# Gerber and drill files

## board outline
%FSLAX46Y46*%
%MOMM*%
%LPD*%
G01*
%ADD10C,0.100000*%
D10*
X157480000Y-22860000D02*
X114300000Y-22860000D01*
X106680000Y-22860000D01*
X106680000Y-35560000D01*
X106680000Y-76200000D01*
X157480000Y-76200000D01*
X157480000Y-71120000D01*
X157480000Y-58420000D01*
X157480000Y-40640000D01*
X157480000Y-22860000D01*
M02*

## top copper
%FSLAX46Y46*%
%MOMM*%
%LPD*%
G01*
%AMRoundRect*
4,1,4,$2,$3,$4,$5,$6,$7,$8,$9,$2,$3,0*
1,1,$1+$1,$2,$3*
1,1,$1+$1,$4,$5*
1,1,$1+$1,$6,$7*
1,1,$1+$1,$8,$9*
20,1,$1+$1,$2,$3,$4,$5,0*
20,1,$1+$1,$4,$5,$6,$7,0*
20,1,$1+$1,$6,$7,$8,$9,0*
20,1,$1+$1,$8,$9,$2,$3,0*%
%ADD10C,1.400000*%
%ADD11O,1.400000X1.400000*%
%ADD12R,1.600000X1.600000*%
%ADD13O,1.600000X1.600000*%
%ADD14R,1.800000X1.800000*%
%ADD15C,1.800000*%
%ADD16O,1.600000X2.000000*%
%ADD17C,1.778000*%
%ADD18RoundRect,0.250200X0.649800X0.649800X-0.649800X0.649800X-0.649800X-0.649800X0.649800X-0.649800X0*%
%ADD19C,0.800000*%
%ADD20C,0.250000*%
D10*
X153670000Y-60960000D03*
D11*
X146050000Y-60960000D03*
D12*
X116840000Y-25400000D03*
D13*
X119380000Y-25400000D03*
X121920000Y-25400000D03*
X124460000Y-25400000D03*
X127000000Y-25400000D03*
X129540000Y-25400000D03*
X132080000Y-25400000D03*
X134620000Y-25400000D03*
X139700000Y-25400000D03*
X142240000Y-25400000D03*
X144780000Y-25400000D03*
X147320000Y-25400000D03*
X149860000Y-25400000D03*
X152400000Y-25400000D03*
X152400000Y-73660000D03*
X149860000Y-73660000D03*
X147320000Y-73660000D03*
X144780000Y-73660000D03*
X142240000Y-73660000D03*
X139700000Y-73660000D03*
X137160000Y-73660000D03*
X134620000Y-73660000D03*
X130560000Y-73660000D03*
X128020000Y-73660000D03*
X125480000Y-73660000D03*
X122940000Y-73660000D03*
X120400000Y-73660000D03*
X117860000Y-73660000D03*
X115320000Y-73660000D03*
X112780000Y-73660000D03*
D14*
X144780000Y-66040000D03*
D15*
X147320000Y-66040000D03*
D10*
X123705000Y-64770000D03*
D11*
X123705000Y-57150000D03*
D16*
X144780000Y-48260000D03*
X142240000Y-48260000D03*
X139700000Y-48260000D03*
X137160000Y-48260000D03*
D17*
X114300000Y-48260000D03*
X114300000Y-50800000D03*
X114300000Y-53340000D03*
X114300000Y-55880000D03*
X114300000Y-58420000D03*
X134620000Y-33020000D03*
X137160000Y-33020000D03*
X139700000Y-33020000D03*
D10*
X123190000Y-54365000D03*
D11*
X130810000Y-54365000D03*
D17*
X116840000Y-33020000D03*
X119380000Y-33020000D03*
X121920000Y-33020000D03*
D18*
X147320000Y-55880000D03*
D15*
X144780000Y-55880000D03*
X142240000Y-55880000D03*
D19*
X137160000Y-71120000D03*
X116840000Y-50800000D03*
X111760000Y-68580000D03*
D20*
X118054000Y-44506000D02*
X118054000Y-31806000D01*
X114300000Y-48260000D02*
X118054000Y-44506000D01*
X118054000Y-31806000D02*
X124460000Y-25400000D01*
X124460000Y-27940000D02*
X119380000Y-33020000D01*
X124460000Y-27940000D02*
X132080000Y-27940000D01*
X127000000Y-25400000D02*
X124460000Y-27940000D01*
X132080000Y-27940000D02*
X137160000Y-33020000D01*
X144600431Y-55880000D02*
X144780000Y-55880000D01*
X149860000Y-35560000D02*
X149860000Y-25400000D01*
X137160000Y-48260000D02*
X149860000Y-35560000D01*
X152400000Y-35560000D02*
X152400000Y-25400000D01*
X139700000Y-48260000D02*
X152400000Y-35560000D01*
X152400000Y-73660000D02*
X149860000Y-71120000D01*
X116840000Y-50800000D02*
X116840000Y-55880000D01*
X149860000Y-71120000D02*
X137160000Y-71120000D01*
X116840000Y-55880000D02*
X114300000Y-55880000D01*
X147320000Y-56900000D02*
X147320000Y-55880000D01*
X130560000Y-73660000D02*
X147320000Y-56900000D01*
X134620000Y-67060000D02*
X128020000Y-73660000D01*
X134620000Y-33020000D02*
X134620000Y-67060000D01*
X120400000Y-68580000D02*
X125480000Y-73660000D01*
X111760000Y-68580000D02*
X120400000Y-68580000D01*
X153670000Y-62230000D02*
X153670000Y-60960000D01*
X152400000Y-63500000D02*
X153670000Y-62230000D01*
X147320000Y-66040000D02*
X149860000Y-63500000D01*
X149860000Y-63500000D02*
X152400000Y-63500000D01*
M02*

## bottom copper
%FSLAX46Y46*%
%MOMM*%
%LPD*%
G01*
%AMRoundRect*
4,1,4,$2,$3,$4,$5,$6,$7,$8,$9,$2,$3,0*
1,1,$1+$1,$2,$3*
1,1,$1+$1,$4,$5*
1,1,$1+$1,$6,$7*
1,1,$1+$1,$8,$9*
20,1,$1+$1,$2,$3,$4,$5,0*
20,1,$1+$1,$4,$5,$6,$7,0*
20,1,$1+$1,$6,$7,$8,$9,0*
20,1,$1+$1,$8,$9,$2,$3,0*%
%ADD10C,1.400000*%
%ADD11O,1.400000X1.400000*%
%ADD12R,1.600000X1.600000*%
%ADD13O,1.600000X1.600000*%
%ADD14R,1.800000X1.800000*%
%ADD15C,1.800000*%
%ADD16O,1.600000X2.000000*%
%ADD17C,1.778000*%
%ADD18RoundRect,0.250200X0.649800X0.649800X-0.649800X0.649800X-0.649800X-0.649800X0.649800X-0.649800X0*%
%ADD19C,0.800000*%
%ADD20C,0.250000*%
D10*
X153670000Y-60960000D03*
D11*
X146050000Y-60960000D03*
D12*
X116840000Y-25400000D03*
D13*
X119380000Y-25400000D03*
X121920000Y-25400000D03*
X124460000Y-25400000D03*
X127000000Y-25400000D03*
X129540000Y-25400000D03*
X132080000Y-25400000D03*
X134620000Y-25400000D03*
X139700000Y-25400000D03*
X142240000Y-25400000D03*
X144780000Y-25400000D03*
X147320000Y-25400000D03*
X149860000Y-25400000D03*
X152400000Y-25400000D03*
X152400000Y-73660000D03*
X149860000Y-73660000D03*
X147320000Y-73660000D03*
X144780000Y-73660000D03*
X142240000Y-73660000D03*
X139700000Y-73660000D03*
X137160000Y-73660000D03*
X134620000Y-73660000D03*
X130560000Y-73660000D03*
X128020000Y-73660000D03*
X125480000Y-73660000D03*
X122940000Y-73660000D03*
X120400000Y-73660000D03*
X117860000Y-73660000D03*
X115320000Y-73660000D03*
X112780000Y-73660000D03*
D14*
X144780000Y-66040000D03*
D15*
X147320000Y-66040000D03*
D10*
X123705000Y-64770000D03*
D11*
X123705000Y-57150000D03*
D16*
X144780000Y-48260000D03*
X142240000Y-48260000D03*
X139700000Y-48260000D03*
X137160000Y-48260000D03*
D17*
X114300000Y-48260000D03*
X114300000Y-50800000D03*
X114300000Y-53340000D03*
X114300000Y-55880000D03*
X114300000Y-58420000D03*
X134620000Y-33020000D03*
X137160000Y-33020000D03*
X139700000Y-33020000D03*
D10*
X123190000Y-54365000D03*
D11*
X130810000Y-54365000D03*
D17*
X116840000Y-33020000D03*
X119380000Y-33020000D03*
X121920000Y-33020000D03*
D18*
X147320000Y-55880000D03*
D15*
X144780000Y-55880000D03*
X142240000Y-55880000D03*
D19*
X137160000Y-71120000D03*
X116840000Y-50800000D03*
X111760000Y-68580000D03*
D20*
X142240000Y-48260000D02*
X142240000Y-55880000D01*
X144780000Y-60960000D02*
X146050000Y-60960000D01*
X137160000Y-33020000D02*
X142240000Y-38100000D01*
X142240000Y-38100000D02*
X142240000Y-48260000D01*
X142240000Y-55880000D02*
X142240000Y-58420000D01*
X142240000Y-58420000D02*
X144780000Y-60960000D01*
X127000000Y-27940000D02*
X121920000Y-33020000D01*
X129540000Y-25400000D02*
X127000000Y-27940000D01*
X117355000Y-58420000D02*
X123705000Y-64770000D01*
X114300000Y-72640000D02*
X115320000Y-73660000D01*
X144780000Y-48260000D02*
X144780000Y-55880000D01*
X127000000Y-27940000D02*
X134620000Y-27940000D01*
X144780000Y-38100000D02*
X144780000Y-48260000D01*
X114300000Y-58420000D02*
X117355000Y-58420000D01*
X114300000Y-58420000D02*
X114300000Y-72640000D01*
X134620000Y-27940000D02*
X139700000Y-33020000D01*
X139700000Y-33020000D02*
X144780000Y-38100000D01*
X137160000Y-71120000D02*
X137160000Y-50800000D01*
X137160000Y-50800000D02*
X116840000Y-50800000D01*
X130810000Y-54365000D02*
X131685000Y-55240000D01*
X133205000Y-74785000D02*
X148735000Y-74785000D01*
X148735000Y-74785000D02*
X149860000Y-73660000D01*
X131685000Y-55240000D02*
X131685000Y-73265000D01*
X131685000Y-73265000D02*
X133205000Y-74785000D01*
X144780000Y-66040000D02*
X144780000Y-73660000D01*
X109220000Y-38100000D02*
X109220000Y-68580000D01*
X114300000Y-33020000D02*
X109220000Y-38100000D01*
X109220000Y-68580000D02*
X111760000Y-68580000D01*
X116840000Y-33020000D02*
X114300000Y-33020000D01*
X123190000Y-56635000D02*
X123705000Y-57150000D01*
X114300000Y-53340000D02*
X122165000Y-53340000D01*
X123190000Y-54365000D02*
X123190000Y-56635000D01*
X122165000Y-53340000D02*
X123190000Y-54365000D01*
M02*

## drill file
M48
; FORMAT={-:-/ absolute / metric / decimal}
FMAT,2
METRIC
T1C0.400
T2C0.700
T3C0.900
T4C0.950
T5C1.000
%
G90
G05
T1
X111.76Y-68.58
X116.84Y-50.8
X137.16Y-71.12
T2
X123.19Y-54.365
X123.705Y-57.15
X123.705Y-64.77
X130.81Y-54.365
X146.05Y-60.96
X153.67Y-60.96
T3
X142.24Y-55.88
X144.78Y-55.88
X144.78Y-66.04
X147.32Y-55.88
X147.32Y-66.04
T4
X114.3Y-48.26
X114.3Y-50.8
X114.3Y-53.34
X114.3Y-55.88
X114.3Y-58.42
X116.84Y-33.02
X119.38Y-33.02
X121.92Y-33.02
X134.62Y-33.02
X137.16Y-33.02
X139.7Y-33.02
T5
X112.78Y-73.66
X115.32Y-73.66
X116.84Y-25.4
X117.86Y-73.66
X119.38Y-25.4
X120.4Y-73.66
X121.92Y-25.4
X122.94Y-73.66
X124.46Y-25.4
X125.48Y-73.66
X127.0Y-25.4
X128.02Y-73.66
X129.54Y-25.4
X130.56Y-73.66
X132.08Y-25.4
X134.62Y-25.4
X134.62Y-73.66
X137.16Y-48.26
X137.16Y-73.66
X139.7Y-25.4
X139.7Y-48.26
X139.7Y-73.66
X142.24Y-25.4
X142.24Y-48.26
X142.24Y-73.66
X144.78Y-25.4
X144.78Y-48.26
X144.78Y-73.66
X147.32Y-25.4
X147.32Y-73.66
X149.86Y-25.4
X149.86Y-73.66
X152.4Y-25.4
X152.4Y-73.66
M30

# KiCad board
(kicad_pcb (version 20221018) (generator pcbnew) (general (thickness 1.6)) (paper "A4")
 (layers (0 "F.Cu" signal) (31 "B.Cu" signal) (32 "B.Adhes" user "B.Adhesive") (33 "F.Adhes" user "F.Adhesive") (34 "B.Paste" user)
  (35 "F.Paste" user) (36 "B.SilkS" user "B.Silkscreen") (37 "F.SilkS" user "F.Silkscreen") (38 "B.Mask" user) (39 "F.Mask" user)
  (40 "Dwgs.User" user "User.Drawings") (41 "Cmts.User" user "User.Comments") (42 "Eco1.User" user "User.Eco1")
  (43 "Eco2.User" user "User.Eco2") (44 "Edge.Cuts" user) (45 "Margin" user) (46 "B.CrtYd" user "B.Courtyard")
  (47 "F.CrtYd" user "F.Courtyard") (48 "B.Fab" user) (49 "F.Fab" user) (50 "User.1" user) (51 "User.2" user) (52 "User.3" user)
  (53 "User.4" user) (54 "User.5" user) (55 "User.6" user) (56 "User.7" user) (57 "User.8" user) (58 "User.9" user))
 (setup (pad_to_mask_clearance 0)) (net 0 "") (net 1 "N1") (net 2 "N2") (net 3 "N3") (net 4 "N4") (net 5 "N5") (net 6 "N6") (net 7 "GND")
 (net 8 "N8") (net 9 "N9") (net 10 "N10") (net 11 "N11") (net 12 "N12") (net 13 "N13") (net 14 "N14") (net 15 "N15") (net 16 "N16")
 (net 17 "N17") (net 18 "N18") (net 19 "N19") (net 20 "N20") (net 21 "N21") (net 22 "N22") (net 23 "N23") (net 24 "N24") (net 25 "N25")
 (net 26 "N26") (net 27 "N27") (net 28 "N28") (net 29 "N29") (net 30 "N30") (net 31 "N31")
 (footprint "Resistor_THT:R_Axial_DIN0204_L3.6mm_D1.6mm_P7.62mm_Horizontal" (layer "F.Cu") (at 153.67 60.96 180)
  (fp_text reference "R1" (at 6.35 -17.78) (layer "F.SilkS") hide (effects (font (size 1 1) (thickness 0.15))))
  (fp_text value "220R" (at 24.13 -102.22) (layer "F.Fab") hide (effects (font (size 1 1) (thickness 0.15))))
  (pad "1" thru_hole circle (at 0 0 180) (size 1.4 1.4) (drill 0.7) (layers "*.Cu" "*.Mask") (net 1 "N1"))
  (pad "2" thru_hole oval (at 7.62 0 180) (size 1.4 1.4) (drill 0.7) (layers "*.Cu" "*.Mask") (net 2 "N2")))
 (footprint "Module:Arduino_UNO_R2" (layer "F.Cu") (at 116.84 25.4)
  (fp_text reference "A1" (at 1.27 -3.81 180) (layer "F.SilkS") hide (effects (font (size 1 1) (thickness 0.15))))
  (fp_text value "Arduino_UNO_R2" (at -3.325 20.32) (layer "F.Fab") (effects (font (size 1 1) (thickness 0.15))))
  (pad "1" thru_hole rect (at 0 0 90) (size 1.6 1.6) (drill 1) (layers "*.Cu" "*.Mask") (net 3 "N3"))
  (pad "2" thru_hole oval (at 2.54 0 90) (size 1.6 1.6) (drill 1) (layers "*.Cu" "*.Mask") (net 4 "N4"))
  (pad "3" thru_hole oval (at 5.08 0 90) (size 1.6 1.6) (drill 1) (layers "*.Cu" "*.Mask") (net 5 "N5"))
  (pad "4" thru_hole oval (at 7.62 0 90) (size 1.6 1.6) (drill 1) (layers "*.Cu" "*.Mask") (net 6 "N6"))
  (pad "5" thru_hole oval (at 10.16 0 90) (size 1.6 1.6) (drill 1) (layers "*.Cu" "*.Mask") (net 2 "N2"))
  (pad "6" thru_hole oval (at 12.7 0 90) (size 1.6 1.6) (drill 1) (layers "*.Cu" "*.Mask") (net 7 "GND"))
  (pad "7" thru_hole oval (at 15.24 0 90) (size 1.6 1.6) (drill 1) (layers "*.Cu" "*.Mask") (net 7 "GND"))
  (pad "8" thru_hole oval (at 17.78 0 90) (size 1.6 1.6) (drill 1) (layers "*.Cu" "*.Mask") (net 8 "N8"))
  (pad "9" thru_hole oval (at 22.86 0 90) (size 1.6 1.6) (drill 1) (layers "*.Cu" "*.Mask") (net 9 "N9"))
  (pad "10" thru_hole oval (at 25.4 0 90) (size 1.6 1.6) (drill 1) (layers "*.Cu" "*.Mask") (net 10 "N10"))
  (pad "11" thru_hole oval (at 27.94 0 90) (size 1.6 1.6) (drill 1) (layers "*.Cu" "*.Mask") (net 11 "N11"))
  (pad "12" thru_hole oval (at 30.48 0 90) (size 1.6 1.6) (drill 1) (layers "*.Cu" "*.Mask") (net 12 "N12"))
  (pad "13" thru_hole oval (at 33.02 0 90) (size 1.6 1.6) (drill 1) (layers "*.Cu" "*.Mask") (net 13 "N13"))
  (pad "14" thru_hole oval (at 35.56 0 90) (size 1.6 1.6) (drill 1) (layers "*.Cu" "*.Mask") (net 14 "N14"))
  (pad "15" thru_hole oval (at 35.56 48.26 90) (size 1.6 1.6) (drill 1) (layers "*.Cu" "*.Mask") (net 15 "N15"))
  (pad "16" thru_hole oval (at 33.02 48.26 90) (size 1.6 1.6) (drill 1) (layers "*.Cu" "*.Mask") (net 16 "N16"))
  (pad "17" thru_hole oval (at 30.48 48.26 90) (size 1.6 1.6) (drill 1) (layers "*.Cu" "*.Mask") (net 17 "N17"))
  (pad "18" thru_hole oval (at 27.94 48.26 90) (size 1.6 1.6) (drill 1) (layers "*.Cu" "*.Mask") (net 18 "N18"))
  (pad "19" thru_hole oval (at 25.4 48.26 90) (size 1.6 1.6) (drill 1) (layers "*.Cu" "*.Mask") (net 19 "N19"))
  (pad "20" thru_hole oval (at 22.86 48.26 90) (size 1.6 1.6) (drill 1) (layers "*.Cu" "*.Mask") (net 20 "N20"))
  (pad "21" thru_hole oval (at 20.32 48.26 90) (size 1.6 1.6) (drill 1) (layers "*.Cu" "*.Mask") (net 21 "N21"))
  (pad "22" thru_hole oval (at 17.78 48.26 90) (size 1.6 1.6) (drill 1) (layers "*.Cu" "*.Mask") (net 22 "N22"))
  (pad "23" thru_hole oval (at 13.72 48.26 90) (size 1.6 1.6) (drill 1) (layers "*.Cu" "*.Mask") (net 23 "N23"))
  (pad "24" thru_hole oval (at 11.18 48.26 90) (size 1.6 1.6) (drill 1) (layers "*.Cu" "*.Mask") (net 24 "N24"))
  (pad "25" thru_hole oval (at 8.64 48.26 90) (size 1.6 1.6) (drill 1) (layers "*.Cu" "*.Mask") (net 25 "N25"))
  (pad "26" thru_hole oval (at 6.1 48.26 90) (size 1.6 1.6) (drill 1) (layers "*.Cu" "*.Mask") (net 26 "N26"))
  (pad "27" thru_hole oval (at 3.56 48.26 90) (size 1.6 1.6) (drill 1) (layers "*.Cu" "*.Mask") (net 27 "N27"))
  (pad "28" thru_hole oval (at 1.02 48.26 90) (size 1.6 1.6) (drill 1) (layers "*.Cu" "*.Mask") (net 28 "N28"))
  (pad "29" thru_hole oval (at -1.52 48.26 90) (size 1.6 1.6) (drill 1) (layers "*.Cu" "*.Mask") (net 7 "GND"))
  (pad "30" thru_hole oval (at -4.06 48.26 90) (size 1.6 1.6) (drill 1) (layers "*.Cu" "*.Mask") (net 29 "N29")))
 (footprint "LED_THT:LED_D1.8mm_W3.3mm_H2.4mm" (layer "F.Cu") (at 144.78 66.04)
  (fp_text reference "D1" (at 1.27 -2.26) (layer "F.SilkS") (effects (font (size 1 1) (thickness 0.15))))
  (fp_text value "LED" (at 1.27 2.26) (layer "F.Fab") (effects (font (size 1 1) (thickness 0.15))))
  (pad "1" thru_hole rect (at 0 0) (size 1.8 1.8) (drill 0.9) (layers "*.Cu" "*.Mask") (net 18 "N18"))
  (pad "2" thru_hole circle (at 2.54 0) (size 1.8 1.8) (drill 0.9) (layers "*.Cu" "*.Mask") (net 1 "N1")))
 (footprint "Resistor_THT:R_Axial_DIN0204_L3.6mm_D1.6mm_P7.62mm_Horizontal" (layer "F.Cu") (at 123.705 64.77 90)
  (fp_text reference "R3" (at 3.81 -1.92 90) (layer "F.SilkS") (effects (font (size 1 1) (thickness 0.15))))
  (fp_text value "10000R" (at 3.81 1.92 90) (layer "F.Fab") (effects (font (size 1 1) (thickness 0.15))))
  (pad "1" thru_hole circle (at 0 0 90) (size 1.4 1.4) (drill 0.7) (layers "*.Cu" "*.Mask") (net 7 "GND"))
  (pad "2" thru_hole oval (at 7.62 0 90) (size 1.4 1.4) (drill 0.7) (layers "*.Cu" "*.Mask") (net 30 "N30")))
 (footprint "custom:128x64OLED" (layer "F.Cu") (at 141.16 37.66 180)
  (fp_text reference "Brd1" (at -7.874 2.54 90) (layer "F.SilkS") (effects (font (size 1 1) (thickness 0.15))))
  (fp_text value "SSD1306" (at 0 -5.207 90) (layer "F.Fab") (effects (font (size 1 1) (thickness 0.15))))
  (pad "1" thru_hole oval (at -3.62 -10.6 270) (size 2 1.6) (drill 1) (layers "*.Cu" "*.Mask") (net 7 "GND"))
  (pad "2" thru_hole oval (at -1.08 -10.6 270) (size 2 1.6) (drill 1) (layers "*.Cu" "*.Mask") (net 2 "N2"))
  (pad "3" thru_hole oval (at 1.46 -10.6 270) (size 2 1.6) (drill 1) (layers "*.Cu" "*.Mask") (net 14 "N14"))
  (pad "4" thru_hole oval (at 4 -10.6 270) (size 2 1.6) (drill 1) (layers "*.Cu" "*.Mask") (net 13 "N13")))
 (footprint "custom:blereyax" (layer "F.Cu") (at 114.3 53.34)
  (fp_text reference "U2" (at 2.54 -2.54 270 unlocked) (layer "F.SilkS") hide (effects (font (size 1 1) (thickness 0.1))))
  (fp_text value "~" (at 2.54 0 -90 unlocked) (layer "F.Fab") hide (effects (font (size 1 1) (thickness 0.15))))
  (pad "1" thru_hole circle (at 0 -5.08) (size 1.778 1.778) (drill 0.95) (layers "*.Cu" "*.Mask") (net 6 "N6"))
  (pad "2" thru_hole circle (at 0 -2.54) (size 1.778 1.778) (drill 0.95) (layers "*.Cu" "*.Mask") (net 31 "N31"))
  (pad "3" thru_hole circle (at 0 0) (size 1.778 1.778) (drill 0.95) (layers "*.Cu" "*.Mask") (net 30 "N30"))
  (pad "4" thru_hole circle (at 0 2.54) (size 1.778 1.778) (drill 0.95) (layers "*.Cu" "*.Mask") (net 15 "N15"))
  (pad "5" thru_hole circle (at 0 5.08) (size 1.778 1.778) (drill 0.95) (layers "*.Cu" "*.Mask") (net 7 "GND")))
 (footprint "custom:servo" (layer "F.Cu") (at 137.16 33.02 90)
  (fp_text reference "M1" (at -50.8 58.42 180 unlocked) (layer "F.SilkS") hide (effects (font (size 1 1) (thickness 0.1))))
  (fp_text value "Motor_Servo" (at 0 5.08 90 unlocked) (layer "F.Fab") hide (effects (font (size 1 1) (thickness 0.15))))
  (pad "1" thru_hole circle (at 0 -2.54 90) (size 1.778 1.778) (drill 0.95) (layers "*.Cu" "*.Mask") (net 24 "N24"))
  (pad "2" thru_hole circle (at 0 0 90) (size 1.778 1.778) (drill 0.95) (layers "*.Cu" "*.Mask") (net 2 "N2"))
  (pad "3" thru_hole circle (at 0 2.54 90) (size 1.778 1.778) (drill 0.95) (layers "*.Cu" "*.Mask") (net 7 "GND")))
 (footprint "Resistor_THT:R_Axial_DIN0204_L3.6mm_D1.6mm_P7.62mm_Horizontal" (layer "F.Cu") (at 123.19 54.365)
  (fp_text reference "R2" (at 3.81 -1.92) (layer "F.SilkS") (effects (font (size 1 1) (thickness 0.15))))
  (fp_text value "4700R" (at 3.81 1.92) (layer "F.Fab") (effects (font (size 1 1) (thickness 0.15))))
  (pad "1" thru_hole circle (at 0 0) (size 1.4 1.4) (drill 0.7) (layers "*.Cu" "*.Mask") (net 30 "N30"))
  (pad "2" thru_hole oval (at 7.62 0) (size 1.4 1.4) (drill 0.7) (layers "*.Cu" "*.Mask") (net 16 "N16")))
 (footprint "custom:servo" (layer "F.Cu") (at 119.38 33.02 90)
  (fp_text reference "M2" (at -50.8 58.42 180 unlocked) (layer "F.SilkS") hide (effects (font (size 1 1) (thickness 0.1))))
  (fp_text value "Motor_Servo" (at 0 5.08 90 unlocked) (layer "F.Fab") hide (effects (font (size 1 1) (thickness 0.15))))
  (pad "1" thru_hole circle (at 0 -2.54 90) (size 1.778 1.778) (drill 0.95) (layers "*.Cu" "*.Mask") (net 25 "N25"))
  (pad "2" thru_hole circle (at 0 0 90) (size 1.778 1.778) (drill 0.95) (layers "*.Cu" "*.Mask") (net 2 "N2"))
  (pad "3" thru_hole circle (at 0 2.54 90) (size 1.778 1.778) (drill 0.95) (layers "*.Cu" "*.Mask") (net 7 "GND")))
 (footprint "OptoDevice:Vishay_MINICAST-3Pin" (layer "F.Cu") (at 147.32 55.88 180)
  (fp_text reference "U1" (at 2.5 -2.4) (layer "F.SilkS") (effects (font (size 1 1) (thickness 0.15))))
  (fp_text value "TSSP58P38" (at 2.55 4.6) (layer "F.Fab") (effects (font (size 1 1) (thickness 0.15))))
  (pad "1" thru_hole roundrect (at 0 0 180) (size 1.8 1.8) (drill 0.9) (layers "*.Cu" "*.Mask") (roundrect_rratio 0.139) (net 23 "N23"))
  (pad "2" thru_hole circle (at 2.54 0 180) (size 1.8 1.8) (drill 0.9) (layers "*.Cu" "*.Mask") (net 7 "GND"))
  (pad "3" thru_hole circle (at 5.08 0 180) (size 1.8 1.8) (drill 0.9) (layers "*.Cu" "*.Mask") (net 2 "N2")))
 (gr_poly
  (pts (xy 157.48 22.86) (xy 114.3 22.86) (xy 106.68 22.86) (xy 106.68 35.56) (xy 106.68 76.2) (xy 157.48 76.2) (xy 157.48 71.12)
   (xy 157.48 58.42) (xy 157.48 40.64))
  (stroke (width 0.1) (type solid)) (fill none) (layer "Edge.Cuts"))
 (segment (start 118.054 44.506) (end 118.054 31.806) (width 0.25) (layer "F.Cu") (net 6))
 (segment (start 114.3 48.26) (end 118.054 44.506) (width 0.25) (layer "F.Cu") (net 6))
 (segment (start 118.054 31.806) (end 124.46 25.4) (width 0.25) (layer "F.Cu") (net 6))
 (segment (start 124.46 27.94) (end 119.38 33.02) (width 0.25) (layer "F.Cu") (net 2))
 (segment (start 124.46 27.94) (end 132.08 27.94) (width 0.25) (layer "F.Cu") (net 2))
 (segment (start 127 25.4) (end 124.46 27.94) (width 0.25) (layer "F.Cu") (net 2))
 (segment (start 132.08 27.94) (end 137.16 33.02) (width 0.25) (layer "F.Cu") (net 2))
 (segment (start 142.24 48.26) (end 142.24 55.88) (width 0.25) (layer "B.Cu") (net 2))
 (segment (start 144.78 60.96) (end 146.05 60.96) (width 0.25) (layer "B.Cu") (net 2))
 (segment (start 137.16 33.02) (end 142.24 38.1) (width 0.25) (layer "B.Cu") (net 2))
 (segment (start 142.24 38.1) (end 142.24 48.26) (width 0.25) (layer "B.Cu") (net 2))
 (segment (start 142.24 55.88) (end 142.24 58.42) (width 0.25) (layer "B.Cu") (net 2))
 (segment (start 142.24 58.42) (end 144.78 60.96) (width 0.25) (layer "B.Cu") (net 2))
 (segment (start 144.600431 55.88) (end 144.78 55.88) (width 0.25) (layer "F.Cu") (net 7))
 (segment (start 127 27.94) (end 121.92 33.02) (width 0.25) (layer "B.Cu") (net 7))
 (segment (start 129.54 25.4) (end 127 27.94) (width 0.25) (layer "B.Cu") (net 7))
 (segment (start 117.355 58.42) (end 123.705 64.77) (width 0.25) (layer "B.Cu") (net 7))
 (segment (start 114.3 72.64) (end 115.32 73.66) (width 0.25) (layer "B.Cu") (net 7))
 (segment (start 144.78 48.26) (end 144.78 55.88) (width 0.25) (layer "B.Cu") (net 7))
 (segment (start 127 27.94) (end 134.62 27.94) (width 0.25) (layer "B.Cu") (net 7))
 (segment (start 144.78 38.1) (end 144.78 48.26) (width 0.25) (layer "B.Cu") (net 7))
 (segment (start 114.3 58.42) (end 117.355 58.42) (width 0.25) (layer "B.Cu") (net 7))
 (segment (start 114.3 58.42) (end 114.3 72.64) (width 0.25) (layer "B.Cu") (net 7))
 (segment (start 134.62 27.94) (end 139.7 33.02) (width 0.25) (layer "B.Cu") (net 7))
 (segment (start 139.7 33.02) (end 144.78 38.1) (width 0.25) (layer "B.Cu") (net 7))
 (segment (start 149.86 35.56) (end 149.86 25.4) (width 0.25) (layer "F.Cu") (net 13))
 (segment (start 137.16 48.26) (end 149.86 35.56) (width 0.25) (layer "F.Cu") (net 13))
 (segment (start 152.4 35.56) (end 152.4 25.4) (width 0.25) (layer "F.Cu") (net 14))
 (segment (start 139.7 48.26) (end 152.4 35.56) (width 0.25) (layer "F.Cu") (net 14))
 (segment (start 152.4 73.66) (end 149.86 71.12) (width 0.25) (layer "F.Cu") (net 15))
 (segment (start 116.84 50.8) (end 116.84 55.88) (width 0.25) (layer "F.Cu") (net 15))
 (segment (start 149.86 71.12) (end 137.16 71.12) (width 0.25) (layer "F.Cu") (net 15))
 (segment (start 116.84 55.88) (end 114.3 55.88) (width 0.25) (layer "F.Cu") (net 15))
 (via (at 137.16 71.12) (size 0.8) (drill 0.4) (layers "F.Cu" "B.Cu") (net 15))
 (via (at 116.84 50.8) (size 0.8) (drill 0.4) (layers "F.Cu" "B.Cu") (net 15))
 (segment (start 137.16 71.12) (end 137.16 50.8) (width 0.25) (layer "B.Cu") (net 15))
 (segment (start 137.16 50.8) (end 116.84 50.8) (width 0.25) (layer "B.Cu") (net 15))
 (segment (start 130.81 54.365) (end 131.685 55.24) (width 0.25) (layer "B.Cu") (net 16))
 (segment (start 133.205 74.785) (end 148.735 74.785) (width 0.25) (layer "B.Cu") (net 16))
 (segment (start 148.735 74.785) (end 149.86 73.66) (width 0.25) (layer "B.Cu") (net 16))
 (segment (start 131.685 55.24) (end 131.685 73.265) (width 0.25) (layer "B.Cu") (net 16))
 (segment (start 131.685 73.265) (end 133.205 74.785) (width 0.25) (layer "B.Cu") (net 16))
 (segment (start 144.78 66.04) (end 144.78 73.66) (width 0.25) (layer "B.Cu") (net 18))
 (segment (start 147.32 56.9) (end 147.32 55.88) (width 0.25) (layer "F.Cu") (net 23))
 (segment (start 130.56 73.66) (end 147.32 56.9) (width 0.25) (layer "F.Cu") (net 23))
 (segment (start 134.62 67.06) (end 128.02 73.66) (width 0.25) (layer "F.Cu") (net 24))
 (segment (start 134.62 33.02) (end 134.62 67.06) (width 0.25) (layer "F.Cu") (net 24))
 (segment (start 120.4 68.58) (end 125.48 73.66) (width 0.25) (layer "F.Cu") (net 25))
 (segment (start 111.76 68.58) (end 120.4 68.58) (width 0.25) (layer "F.Cu") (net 25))
 (via (at 111.76 68.58) (size 0.8) (drill 0.4) (layers "F.Cu" "B.Cu") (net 25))
 (segment (start 109.22 38.1) (end 109.22 68.58) (width 0.25) (layer "B.Cu") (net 25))
 (segment (start 114.3 33.02) (end 109.22 38.1) (width 0.25) (layer "B.Cu") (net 25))
 (segment (start 109.22 68.58) (end 111.76 68.58) (width 0.25) (layer "B.Cu") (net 25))
 (segment (start 116.84 33.02) (end 114.3 33.02) (width 0.25) (layer "B.Cu") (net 25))
 (segment (start 153.67 62.23) (end 153.67 60.96) (width 0.25) (layer "F.Cu") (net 1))
 (segment (start 152.4 63.5) (end 153.67 62.23) (width 0.25) (layer "F.Cu") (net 1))
 (segment (start 147.32 66.04) (end 149.86 63.5) (width 0.25) (layer "F.Cu") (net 1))
 (segment (start 149.86 63.5) (end 152.4 63.5) (width 0.25) (layer "F.Cu") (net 1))
 (segment (start 123.19 56.635) (end 123.705 57.15) (width 0.25) (layer "B.Cu") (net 30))
 (segment (start 114.3 53.34) (end 122.165 53.34) (width 0.25) (layer "B.Cu") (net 30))
 (segment (start 123.19 54.365) (end 123.19 56.635) (width 0.25) (layer "B.Cu") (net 30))
 (segment (start 122.165 53.34) (end 123.19 54.365) (width 0.25) (layer "B.Cu") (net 30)))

